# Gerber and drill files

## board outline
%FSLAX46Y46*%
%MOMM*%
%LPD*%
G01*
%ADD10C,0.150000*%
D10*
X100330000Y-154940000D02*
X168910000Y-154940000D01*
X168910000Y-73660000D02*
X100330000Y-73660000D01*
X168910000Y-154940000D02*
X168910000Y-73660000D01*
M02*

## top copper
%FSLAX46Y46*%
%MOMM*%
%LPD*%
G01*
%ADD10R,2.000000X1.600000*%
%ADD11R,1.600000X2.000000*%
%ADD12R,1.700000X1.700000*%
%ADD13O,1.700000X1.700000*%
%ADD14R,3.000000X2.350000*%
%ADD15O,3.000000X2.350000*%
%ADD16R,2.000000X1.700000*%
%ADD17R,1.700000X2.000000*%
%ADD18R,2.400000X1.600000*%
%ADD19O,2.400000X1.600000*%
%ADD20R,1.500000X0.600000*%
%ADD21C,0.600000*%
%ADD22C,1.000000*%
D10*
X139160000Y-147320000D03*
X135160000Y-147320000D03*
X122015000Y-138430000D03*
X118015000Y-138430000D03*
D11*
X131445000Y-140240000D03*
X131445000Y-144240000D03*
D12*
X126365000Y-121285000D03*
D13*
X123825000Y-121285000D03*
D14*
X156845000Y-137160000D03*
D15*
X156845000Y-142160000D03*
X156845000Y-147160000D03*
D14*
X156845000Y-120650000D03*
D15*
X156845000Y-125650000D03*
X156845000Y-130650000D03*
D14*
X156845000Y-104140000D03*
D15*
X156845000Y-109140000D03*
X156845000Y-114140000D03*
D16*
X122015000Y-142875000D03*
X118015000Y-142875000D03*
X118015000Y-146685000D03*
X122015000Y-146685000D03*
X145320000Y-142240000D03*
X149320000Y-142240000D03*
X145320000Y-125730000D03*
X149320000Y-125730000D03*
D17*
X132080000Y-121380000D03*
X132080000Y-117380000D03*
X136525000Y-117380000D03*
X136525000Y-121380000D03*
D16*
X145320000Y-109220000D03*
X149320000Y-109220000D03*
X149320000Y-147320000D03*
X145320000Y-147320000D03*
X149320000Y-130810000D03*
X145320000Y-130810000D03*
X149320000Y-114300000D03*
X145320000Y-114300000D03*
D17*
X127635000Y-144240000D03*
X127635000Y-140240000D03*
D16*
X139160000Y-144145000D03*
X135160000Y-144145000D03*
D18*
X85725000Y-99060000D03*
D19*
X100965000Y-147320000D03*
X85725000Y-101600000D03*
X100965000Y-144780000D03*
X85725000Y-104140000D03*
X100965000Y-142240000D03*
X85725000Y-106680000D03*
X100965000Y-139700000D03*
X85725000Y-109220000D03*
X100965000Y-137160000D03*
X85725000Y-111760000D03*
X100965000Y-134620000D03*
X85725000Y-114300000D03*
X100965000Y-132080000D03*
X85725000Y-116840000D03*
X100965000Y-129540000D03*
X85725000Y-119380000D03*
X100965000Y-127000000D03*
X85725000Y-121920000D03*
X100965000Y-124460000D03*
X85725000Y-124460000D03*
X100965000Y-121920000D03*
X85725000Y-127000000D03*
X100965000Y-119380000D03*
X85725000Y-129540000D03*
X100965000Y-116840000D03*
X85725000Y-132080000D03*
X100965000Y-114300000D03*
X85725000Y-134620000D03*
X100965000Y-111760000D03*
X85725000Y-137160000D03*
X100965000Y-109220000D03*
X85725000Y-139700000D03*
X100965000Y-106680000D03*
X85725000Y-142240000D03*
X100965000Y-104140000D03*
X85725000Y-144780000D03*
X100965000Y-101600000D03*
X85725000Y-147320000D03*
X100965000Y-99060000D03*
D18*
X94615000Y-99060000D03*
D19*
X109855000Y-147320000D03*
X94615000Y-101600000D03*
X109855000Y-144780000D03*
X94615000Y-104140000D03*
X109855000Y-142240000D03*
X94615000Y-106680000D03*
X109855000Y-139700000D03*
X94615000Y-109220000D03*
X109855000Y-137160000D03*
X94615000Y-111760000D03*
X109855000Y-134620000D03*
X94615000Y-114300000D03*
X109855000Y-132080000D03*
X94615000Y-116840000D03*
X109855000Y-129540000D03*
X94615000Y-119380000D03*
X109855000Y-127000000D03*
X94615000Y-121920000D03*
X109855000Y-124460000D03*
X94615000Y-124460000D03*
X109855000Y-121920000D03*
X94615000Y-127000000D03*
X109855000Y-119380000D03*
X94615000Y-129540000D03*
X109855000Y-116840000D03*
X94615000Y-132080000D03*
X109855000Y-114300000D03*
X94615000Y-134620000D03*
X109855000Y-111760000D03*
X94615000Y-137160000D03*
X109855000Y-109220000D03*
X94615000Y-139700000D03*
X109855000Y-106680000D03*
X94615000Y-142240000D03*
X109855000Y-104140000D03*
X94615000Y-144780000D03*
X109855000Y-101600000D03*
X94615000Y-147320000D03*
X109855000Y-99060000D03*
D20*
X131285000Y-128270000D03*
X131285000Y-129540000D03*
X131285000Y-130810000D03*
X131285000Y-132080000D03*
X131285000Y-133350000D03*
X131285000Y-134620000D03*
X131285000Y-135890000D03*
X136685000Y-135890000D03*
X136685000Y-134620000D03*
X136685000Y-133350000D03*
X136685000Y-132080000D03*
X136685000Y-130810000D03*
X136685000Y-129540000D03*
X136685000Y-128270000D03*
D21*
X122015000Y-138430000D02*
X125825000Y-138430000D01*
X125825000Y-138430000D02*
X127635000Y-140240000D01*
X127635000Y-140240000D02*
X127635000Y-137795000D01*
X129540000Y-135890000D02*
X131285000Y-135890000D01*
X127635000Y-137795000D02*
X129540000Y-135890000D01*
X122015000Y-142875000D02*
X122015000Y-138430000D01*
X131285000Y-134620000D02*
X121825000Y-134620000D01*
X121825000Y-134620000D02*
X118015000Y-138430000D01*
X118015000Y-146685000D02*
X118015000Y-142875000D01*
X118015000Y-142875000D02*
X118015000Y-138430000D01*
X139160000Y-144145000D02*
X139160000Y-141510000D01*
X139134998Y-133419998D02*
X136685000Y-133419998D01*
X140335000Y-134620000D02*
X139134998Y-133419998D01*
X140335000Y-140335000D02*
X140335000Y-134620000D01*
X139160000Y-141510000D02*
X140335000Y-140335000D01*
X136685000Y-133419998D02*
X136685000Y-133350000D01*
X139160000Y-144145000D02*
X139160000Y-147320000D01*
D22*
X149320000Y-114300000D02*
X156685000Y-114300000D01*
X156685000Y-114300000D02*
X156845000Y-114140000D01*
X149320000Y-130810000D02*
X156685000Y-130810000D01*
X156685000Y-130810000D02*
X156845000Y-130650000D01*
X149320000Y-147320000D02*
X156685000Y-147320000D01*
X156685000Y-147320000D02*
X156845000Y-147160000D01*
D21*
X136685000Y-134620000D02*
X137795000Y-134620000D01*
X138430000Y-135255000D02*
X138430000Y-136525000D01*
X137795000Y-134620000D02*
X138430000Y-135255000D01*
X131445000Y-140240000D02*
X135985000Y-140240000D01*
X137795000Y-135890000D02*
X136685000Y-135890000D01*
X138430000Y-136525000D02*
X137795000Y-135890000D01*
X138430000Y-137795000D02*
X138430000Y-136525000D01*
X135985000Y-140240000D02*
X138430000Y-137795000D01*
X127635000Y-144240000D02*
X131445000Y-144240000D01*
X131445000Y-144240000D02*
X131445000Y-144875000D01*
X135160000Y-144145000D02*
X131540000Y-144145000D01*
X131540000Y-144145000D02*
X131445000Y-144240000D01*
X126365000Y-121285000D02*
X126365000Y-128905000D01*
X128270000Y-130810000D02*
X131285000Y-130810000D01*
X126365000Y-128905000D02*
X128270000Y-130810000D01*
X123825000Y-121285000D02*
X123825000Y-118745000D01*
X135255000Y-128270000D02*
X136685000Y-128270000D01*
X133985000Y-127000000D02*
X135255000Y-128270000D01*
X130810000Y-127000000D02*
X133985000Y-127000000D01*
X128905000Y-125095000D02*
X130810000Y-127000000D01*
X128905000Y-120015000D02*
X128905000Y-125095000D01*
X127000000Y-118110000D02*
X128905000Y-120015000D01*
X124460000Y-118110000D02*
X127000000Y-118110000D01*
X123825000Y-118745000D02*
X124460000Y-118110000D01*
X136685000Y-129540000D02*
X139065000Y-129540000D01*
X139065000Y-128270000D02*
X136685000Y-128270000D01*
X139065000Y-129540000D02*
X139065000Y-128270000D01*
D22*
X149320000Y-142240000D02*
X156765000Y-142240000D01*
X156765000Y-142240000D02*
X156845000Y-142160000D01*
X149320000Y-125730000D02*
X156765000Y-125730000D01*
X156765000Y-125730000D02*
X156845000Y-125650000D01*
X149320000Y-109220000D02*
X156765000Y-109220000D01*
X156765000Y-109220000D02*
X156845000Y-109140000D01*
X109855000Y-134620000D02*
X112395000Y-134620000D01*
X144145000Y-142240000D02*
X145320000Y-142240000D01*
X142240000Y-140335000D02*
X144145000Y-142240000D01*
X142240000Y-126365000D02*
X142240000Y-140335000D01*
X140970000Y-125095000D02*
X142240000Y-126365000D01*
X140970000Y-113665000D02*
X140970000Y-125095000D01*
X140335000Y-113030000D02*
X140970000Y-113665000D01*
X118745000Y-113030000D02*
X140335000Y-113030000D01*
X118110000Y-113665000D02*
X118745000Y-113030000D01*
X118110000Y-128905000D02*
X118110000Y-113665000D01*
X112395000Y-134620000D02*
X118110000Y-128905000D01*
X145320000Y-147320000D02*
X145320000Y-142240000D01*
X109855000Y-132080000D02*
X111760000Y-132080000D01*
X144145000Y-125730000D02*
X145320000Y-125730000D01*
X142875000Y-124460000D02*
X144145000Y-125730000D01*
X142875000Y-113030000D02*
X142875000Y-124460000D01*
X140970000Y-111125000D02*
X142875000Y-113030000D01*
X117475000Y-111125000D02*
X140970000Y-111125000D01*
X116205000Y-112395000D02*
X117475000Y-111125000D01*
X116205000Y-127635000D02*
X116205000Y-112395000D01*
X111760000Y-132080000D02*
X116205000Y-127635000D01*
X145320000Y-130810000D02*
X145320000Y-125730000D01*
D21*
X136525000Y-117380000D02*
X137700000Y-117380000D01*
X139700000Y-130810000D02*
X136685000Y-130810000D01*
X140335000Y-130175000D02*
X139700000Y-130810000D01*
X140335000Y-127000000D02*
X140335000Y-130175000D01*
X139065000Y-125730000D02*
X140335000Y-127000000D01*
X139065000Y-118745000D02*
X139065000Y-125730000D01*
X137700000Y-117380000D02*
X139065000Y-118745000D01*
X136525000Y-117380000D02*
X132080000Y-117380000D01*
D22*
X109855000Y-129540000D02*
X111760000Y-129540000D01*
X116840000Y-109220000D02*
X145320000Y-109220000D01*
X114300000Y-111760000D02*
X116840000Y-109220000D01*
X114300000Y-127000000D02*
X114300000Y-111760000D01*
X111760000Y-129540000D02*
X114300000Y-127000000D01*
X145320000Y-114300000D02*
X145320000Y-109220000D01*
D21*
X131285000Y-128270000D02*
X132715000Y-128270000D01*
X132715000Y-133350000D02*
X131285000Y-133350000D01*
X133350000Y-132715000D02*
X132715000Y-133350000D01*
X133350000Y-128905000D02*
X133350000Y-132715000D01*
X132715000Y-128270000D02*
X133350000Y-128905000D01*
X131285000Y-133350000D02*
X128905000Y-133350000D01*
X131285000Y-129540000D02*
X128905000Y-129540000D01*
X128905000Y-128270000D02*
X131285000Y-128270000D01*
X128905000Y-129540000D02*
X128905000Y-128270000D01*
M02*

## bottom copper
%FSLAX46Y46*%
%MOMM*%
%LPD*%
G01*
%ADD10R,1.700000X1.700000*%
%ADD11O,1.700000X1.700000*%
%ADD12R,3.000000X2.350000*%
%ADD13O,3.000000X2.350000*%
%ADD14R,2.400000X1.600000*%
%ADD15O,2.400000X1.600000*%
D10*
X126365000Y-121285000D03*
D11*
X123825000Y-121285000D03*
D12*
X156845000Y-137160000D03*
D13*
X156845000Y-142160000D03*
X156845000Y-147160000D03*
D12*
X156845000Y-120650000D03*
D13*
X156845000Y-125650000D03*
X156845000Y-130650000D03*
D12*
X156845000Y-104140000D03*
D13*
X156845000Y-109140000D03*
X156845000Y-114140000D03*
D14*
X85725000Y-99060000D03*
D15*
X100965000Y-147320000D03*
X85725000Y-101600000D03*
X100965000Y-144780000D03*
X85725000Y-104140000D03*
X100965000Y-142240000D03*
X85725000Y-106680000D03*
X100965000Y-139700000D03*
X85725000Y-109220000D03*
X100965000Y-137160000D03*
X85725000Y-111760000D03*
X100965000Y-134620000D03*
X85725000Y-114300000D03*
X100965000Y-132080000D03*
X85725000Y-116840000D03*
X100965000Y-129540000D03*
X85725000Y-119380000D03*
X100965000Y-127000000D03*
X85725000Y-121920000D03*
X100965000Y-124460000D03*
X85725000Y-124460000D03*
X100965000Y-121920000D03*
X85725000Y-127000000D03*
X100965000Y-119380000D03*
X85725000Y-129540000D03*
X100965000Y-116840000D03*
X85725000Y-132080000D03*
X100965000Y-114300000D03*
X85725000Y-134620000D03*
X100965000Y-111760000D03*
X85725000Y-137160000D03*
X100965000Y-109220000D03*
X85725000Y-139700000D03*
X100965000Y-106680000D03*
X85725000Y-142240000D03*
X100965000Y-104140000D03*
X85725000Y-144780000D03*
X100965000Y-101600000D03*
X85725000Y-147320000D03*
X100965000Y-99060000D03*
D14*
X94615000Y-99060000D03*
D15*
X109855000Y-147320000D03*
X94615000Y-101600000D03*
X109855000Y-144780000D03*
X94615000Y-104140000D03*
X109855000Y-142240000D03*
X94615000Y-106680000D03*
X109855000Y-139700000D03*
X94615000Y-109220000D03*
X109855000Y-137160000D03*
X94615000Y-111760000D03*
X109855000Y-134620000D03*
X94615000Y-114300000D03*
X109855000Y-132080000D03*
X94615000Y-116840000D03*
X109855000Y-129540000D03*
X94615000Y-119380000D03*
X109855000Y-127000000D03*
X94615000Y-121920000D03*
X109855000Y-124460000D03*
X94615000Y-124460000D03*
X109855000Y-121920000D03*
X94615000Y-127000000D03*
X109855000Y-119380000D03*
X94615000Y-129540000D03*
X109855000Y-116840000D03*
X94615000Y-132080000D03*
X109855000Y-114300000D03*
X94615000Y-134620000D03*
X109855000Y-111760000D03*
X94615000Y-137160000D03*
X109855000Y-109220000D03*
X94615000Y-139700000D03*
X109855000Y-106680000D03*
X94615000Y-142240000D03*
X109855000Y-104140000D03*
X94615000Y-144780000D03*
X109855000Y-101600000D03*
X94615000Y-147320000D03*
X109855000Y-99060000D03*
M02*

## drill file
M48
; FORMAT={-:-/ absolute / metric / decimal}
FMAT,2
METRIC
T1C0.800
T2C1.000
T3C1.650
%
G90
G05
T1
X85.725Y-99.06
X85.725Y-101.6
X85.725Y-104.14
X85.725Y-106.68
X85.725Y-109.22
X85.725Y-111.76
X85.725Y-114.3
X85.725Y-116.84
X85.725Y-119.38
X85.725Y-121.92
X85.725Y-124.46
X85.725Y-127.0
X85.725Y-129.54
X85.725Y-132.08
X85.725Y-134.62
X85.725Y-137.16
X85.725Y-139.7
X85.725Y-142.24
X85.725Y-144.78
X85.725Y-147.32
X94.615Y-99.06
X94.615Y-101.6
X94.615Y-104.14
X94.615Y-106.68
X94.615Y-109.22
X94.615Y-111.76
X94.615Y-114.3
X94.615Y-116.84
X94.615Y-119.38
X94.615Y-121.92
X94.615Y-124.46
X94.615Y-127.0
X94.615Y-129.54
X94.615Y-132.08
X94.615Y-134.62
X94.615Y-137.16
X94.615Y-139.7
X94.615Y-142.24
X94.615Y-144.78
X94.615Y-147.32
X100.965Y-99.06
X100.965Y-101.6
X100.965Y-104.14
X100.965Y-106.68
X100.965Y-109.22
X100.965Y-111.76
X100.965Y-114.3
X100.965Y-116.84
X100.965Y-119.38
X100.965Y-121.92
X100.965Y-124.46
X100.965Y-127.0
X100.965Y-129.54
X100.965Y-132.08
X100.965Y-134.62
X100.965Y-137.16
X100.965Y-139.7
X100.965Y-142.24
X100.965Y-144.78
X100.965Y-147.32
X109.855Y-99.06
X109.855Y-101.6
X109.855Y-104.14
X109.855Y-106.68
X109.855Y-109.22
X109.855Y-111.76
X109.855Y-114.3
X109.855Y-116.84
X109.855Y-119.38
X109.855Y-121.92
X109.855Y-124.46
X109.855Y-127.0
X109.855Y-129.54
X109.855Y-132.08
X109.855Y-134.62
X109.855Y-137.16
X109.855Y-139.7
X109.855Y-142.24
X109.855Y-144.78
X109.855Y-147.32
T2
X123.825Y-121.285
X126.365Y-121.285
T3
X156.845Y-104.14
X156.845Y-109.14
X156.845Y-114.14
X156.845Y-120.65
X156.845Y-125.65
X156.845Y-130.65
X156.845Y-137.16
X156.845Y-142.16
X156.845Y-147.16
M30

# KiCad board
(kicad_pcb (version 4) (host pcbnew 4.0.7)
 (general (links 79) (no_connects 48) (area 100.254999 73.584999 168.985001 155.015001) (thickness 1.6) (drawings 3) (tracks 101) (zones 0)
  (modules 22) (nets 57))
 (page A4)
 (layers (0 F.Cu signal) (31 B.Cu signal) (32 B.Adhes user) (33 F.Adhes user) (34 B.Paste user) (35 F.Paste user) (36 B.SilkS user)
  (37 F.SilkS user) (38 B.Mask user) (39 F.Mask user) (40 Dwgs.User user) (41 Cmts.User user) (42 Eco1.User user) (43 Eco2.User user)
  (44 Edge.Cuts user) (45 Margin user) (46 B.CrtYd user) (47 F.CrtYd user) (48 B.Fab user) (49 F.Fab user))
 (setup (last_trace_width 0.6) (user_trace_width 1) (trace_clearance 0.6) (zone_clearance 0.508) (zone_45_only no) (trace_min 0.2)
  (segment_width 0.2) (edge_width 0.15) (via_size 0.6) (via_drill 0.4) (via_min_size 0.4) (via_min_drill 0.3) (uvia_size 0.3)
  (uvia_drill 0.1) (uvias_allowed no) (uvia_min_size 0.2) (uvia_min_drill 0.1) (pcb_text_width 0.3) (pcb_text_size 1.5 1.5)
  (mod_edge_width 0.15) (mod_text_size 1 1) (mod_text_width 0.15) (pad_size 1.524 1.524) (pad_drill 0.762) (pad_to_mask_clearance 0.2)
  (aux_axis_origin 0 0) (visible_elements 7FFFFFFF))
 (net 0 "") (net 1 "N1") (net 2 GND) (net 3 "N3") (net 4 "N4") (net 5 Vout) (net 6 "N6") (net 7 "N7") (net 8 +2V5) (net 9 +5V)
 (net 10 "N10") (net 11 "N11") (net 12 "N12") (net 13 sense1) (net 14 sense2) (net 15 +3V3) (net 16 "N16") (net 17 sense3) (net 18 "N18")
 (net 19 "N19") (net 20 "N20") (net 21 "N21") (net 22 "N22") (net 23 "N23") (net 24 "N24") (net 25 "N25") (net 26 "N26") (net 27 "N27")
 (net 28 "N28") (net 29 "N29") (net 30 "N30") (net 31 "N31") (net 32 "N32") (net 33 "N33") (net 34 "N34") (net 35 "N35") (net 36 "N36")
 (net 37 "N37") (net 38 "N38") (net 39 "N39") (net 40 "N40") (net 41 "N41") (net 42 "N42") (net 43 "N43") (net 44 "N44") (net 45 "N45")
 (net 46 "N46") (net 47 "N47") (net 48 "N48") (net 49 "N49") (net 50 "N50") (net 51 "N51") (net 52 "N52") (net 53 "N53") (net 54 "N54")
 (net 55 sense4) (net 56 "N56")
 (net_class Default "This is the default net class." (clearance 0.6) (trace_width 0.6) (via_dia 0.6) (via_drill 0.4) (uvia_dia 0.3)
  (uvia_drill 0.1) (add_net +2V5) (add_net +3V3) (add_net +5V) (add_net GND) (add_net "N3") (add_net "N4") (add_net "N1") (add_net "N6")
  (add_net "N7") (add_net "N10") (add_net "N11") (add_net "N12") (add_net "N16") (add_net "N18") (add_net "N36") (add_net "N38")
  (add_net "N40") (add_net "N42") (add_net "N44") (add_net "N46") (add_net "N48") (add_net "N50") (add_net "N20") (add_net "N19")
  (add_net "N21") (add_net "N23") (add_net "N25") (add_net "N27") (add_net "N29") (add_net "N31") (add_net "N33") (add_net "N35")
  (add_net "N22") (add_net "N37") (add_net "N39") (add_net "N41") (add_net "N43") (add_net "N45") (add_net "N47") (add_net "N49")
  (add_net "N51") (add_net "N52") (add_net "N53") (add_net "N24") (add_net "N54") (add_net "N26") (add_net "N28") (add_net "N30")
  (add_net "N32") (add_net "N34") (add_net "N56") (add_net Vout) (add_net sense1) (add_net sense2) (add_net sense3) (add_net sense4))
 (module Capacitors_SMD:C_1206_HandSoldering (layer F.Cu) (at 137.16 147.32 180)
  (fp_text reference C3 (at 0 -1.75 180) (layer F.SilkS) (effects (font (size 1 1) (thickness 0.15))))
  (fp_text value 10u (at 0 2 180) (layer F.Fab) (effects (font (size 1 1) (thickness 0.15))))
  (pad 1 smd rect (at -2 0 180) (size 2 1.6) (layers F.Cu F.Paste F.Mask) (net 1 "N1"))
  (pad 2 smd rect (at 2 0 180) (size 2 1.6) (layers F.Cu F.Paste F.Mask) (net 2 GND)))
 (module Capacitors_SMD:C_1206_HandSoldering (layer F.Cu) (at 120.015 138.43 180)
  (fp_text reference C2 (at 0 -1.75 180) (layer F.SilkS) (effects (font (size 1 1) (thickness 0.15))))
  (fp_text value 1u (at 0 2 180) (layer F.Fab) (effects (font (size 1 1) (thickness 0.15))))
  (pad 1 smd rect (at -2 0 180) (size 2 1.6) (layers F.Cu F.Paste F.Mask) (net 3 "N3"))
  (pad 2 smd rect (at 2 0 180) (size 2 1.6) (layers F.Cu F.Paste F.Mask) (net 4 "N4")))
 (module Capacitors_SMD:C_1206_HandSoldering (layer F.Cu) (at 131.445 142.24 270)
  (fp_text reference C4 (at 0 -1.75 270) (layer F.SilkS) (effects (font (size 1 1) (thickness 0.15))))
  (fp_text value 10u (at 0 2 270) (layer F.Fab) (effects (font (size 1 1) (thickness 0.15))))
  (pad 1 smd rect (at -2 0 270) (size 2 1.6) (layers F.Cu F.Paste F.Mask) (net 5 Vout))
  (pad 2 smd rect (at 2 0 270) (size 2 1.6) (layers F.Cu F.Paste F.Mask) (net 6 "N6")))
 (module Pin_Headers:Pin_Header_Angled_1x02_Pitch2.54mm (layer B.Cu) (at 126.365 121.285 90)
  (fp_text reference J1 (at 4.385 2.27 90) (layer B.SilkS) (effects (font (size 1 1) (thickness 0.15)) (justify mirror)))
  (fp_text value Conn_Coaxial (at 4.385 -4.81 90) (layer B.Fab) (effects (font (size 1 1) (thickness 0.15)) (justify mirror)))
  (pad 1 thru_hole rect (at 0 0 90) (size 1.7 1.7) (drill 1) (layers *.Cu *.Mask) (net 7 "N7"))
  (pad 2 thru_hole oval (at 0 -2.54 90) (size 1.7 1.7) (drill 1) (layers *.Cu *.Mask) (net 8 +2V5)))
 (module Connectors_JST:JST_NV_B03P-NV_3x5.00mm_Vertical (layer F.Cu) (at 156.845 137.16 270)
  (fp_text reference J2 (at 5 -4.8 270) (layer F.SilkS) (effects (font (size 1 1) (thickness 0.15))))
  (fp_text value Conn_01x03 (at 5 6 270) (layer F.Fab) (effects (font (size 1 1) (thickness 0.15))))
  (pad 1 thru_hole rect (at 0 0 270) (size 2.35 3) (drill 1.65) (layers *.Cu *.Mask) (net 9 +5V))
  (pad 2 thru_hole oval (at 5 0 270) (size 2.35 3) (drill 1.65) (layers *.Cu *.Mask) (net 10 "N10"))
  (pad 3 thru_hole oval (at 10 0 270) (size 2.35 3) (drill 1.65) (layers *.Cu *.Mask) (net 2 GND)))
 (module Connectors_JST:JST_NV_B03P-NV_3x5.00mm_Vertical (layer F.Cu) (at 156.845 120.65 270)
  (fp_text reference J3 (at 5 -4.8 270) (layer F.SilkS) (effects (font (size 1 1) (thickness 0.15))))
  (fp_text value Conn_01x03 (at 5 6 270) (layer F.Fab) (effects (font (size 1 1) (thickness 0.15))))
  (pad 1 thru_hole rect (at 0 0 270) (size 2.35 3) (drill 1.65) (layers *.Cu *.Mask) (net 9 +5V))
  (pad 2 thru_hole oval (at 5 0 270) (size 2.35 3) (drill 1.65) (layers *.Cu *.Mask) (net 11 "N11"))
  (pad 3 thru_hole oval (at 10 0 270) (size 2.35 3) (drill 1.65) (layers *.Cu *.Mask) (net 2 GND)))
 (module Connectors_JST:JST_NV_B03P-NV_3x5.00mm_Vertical (layer F.Cu) (at 156.845 104.14 270)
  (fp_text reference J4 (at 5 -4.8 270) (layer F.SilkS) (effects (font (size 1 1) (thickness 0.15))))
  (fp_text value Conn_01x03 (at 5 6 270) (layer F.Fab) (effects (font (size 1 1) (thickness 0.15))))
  (pad 1 thru_hole rect (at 0 0 270) (size 2.35 3) (drill 1.65) (layers *.Cu *.Mask) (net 9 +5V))
  (pad 2 thru_hole oval (at 5 0 270) (size 2.35 3) (drill 1.65) (layers *.Cu *.Mask) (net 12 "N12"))
  (pad 3 thru_hole oval (at 10 0 270) (size 2.35 3) (drill 1.65) (layers *.Cu *.Mask) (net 2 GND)))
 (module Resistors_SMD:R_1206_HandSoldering (layer F.Cu) (at 120.015 142.875 180)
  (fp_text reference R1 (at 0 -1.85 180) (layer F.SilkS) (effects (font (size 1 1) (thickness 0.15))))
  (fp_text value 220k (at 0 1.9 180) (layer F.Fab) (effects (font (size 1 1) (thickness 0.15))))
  (pad 1 smd rect (at -2 0 180) (size 2 1.7) (layers F.Cu F.Paste F.Mask) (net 3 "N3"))
  (pad 2 smd rect (at 2 0 180) (size 2 1.7) (layers F.Cu F.Paste F.Mask) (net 4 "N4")))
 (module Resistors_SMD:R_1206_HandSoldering (layer F.Cu) (at 120.015 146.685)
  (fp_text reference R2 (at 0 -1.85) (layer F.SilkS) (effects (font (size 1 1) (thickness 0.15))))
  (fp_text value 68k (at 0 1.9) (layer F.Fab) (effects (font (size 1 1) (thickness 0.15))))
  (pad 1 smd rect (at -2 0) (size 2 1.7) (layers F.Cu F.Paste F.Mask) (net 4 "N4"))
  (pad 2 smd rect (at 2 0) (size 2 1.7) (layers F.Cu F.Paste F.Mask) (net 8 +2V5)))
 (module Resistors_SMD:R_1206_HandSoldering (layer F.Cu) (at 147.32 142.24)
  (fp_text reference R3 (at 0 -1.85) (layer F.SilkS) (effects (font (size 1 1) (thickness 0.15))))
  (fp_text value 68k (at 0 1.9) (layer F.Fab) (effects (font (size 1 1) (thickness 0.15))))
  (pad 1 smd rect (at -2 0) (size 2 1.7) (layers F.Cu F.Paste F.Mask) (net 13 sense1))
  (pad 2 smd rect (at 2 0) (size 2 1.7) (layers F.Cu F.Paste F.Mask) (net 10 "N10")))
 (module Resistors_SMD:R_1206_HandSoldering (layer F.Cu) (at 147.32 125.73)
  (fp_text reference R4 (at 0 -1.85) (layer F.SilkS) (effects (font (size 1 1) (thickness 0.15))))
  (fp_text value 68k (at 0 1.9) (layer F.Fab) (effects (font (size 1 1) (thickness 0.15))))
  (pad 1 smd rect (at -2 0) (size 2 1.7) (layers F.Cu F.Paste F.Mask) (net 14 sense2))
  (pad 2 smd rect (at 2 0) (size 2 1.7) (layers F.Cu F.Paste F.Mask) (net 11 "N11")))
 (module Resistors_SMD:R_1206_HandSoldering (layer F.Cu) (at 132.08 119.38 90)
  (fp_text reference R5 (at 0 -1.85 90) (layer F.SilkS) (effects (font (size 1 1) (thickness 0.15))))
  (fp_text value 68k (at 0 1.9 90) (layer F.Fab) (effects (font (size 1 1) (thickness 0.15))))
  (pad 1 smd rect (at -2 0 90) (size 2 1.7) (layers F.Cu F.Paste F.Mask) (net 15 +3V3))
  (pad 2 smd rect (at 2 0 90) (size 2 1.7) (layers F.Cu F.Paste F.Mask) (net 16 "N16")))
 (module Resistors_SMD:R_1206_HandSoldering (layer F.Cu) (at 136.525 119.38 270)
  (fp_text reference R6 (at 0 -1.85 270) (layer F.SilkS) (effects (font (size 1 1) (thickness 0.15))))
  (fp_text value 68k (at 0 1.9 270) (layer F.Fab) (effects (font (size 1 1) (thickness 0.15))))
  (pad 1 smd rect (at -2 0 270) (size 2 1.7) (layers F.Cu F.Paste F.Mask) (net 16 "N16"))
  (pad 2 smd rect (at 2 0 270) (size 2 1.7) (layers F.Cu F.Paste F.Mask) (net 2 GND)))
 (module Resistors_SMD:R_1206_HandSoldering (layer F.Cu) (at 147.32 109.22)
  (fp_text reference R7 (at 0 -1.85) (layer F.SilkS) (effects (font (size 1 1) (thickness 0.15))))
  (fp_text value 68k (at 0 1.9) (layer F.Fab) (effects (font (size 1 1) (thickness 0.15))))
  (pad 1 smd rect (at -2 0) (size 2 1.7) (layers F.Cu F.Paste F.Mask) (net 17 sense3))
  (pad 2 smd rect (at 2 0) (size 2 1.7) (layers F.Cu F.Paste F.Mask) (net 12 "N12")))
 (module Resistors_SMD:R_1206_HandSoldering (layer F.Cu) (at 147.32 147.32 180)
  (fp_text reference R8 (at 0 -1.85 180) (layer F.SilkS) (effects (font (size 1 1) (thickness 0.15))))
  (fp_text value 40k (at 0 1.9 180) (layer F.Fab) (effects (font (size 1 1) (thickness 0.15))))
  (pad 1 smd rect (at -2 0 180) (size 2 1.7) (layers F.Cu F.Paste F.Mask) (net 2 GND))
  (pad 2 smd rect (at 2 0 180) (size 2 1.7) (layers F.Cu F.Paste F.Mask) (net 13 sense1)))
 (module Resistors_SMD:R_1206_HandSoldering (layer F.Cu) (at 147.32 130.81 180)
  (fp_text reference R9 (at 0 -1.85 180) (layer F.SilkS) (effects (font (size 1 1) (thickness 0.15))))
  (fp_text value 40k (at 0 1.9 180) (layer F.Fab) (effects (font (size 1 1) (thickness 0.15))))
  (pad 1 smd rect (at -2 0 180) (size 2 1.7) (layers F.Cu F.Paste F.Mask) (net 2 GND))
  (pad 2 smd rect (at 2 0 180) (size 2 1.7) (layers F.Cu F.Paste F.Mask) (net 14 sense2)))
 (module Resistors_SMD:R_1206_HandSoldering (layer F.Cu) (at 147.32 114.3 180)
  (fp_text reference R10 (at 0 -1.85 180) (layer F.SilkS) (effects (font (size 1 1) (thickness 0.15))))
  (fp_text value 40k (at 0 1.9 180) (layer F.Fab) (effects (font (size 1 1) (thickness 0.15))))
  (pad 1 smd rect (at -2 0 180) (size 2 1.7) (layers F.Cu F.Paste F.Mask) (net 2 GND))
  (pad 2 smd rect (at 2 0 180) (size 2 1.7) (layers F.Cu F.Paste F.Mask) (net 17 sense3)))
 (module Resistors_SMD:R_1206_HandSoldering (layer F.Cu) (at 127.635 142.24 90)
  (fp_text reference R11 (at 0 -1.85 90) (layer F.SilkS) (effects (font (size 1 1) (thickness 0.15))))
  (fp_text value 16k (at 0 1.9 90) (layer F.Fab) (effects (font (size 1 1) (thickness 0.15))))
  (pad 1 smd rect (at -2 0 90) (size 2 1.7) (layers F.Cu F.Paste F.Mask) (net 6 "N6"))
  (pad 2 smd rect (at 2 0 90) (size 2 1.7) (layers F.Cu F.Paste F.Mask) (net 3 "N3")))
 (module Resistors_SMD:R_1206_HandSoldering (layer F.Cu) (at 137.16 144.145 180)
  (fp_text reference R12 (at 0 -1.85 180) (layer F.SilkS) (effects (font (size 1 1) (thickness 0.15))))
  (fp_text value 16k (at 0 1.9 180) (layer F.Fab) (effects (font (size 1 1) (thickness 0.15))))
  (pad 1 smd rect (at -2 0 180) (size 2 1.7) (layers F.Cu F.Paste F.Mask) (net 1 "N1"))
  (pad 2 smd rect (at 2 0 180) (size 2 1.7) (layers F.Cu F.Paste F.Mask) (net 6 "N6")))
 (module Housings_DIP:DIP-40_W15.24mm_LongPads (layer F.Cu) (at 85.725 99.06)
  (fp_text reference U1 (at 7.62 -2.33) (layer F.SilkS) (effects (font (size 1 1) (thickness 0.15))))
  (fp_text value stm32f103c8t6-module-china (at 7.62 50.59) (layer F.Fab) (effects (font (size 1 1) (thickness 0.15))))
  (pad 1 thru_hole rect (at 0 0) (size 2.4 1.6) (drill 0.8) (layers *.Cu *.Mask) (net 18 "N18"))
  (pad 21 thru_hole oval (at 15.24 48.26) (size 2.4 1.6) (drill 0.8) (layers *.Cu *.Mask) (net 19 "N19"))
  (pad 2 thru_hole oval (at 0 2.54) (size 2.4 1.6) (drill 0.8) (layers *.Cu *.Mask) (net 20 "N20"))
  (pad 22 thru_hole oval (at 15.24 45.72) (size 2.4 1.6) (drill 0.8) (layers *.Cu *.Mask) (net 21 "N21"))
  (pad 3 thru_hole oval (at 0 5.08) (size 2.4 1.6) (drill 0.8) (layers *.Cu *.Mask) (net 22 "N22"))
  (pad 23 thru_hole oval (at 15.24 43.18) (size 2.4 1.6) (drill 0.8) (layers *.Cu *.Mask) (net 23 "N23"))
  (pad 4 thru_hole oval (at 0 7.62) (size 2.4 1.6) (drill 0.8) (layers *.Cu *.Mask) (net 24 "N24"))
  (pad 24 thru_hole oval (at 15.24 40.64) (size 2.4 1.6) (drill 0.8) (layers *.Cu *.Mask) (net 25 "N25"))
  (pad 5 thru_hole oval (at 0 10.16) (size 2.4 1.6) (drill 0.8) (layers *.Cu *.Mask) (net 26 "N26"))
  (pad 25 thru_hole oval (at 15.24 38.1) (size 2.4 1.6) (drill 0.8) (layers *.Cu *.Mask) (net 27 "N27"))
  (pad 6 thru_hole oval (at 0 12.7) (size 2.4 1.6) (drill 0.8) (layers *.Cu *.Mask) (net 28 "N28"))
  (pad 26 thru_hole oval (at 15.24 35.56) (size 2.4 1.6) (drill 0.8) (layers *.Cu *.Mask) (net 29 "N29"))
  (pad 7 thru_hole oval (at 0 15.24) (size 2.4 1.6) (drill 0.8) (layers *.Cu *.Mask) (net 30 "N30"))
  (pad 27 thru_hole oval (at 15.24 33.02) (size 2.4 1.6) (drill 0.8) (layers *.Cu *.Mask) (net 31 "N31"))
  (pad 8 thru_hole oval (at 0 17.78) (size 2.4 1.6) (drill 0.8) (layers *.Cu *.Mask) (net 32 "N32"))
  (pad 28 thru_hole oval (at 15.24 30.48) (size 2.4 1.6) (drill 0.8) (layers *.Cu *.Mask) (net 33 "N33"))
  (pad 9 thru_hole oval (at 0 20.32) (size 2.4 1.6) (drill 0.8) (layers *.Cu *.Mask) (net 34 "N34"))
  (pad 29 thru_hole oval (at 15.24 27.94) (size 2.4 1.6) (drill 0.8) (layers *.Cu *.Mask) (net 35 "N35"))
  (pad 10 thru_hole oval (at 0 22.86) (size 2.4 1.6) (drill 0.8) (layers *.Cu *.Mask) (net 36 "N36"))
  (pad 30 thru_hole oval (at 15.24 25.4) (size 2.4 1.6) (drill 0.8) (layers *.Cu *.Mask) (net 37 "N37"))
  (pad 11 thru_hole oval (at 0 25.4) (size 2.4 1.6) (drill 0.8) (layers *.Cu *.Mask) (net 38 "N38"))
  (pad 31 thru_hole oval (at 15.24 22.86) (size 2.4 1.6) (drill 0.8) (layers *.Cu *.Mask) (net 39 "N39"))
  (pad 12 thru_hole oval (at 0 27.94) (size 2.4 1.6) (drill 0.8) (layers *.Cu *.Mask) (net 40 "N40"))
  (pad 32 thru_hole oval (at 15.24 20.32) (size 2.4 1.6) (drill 0.8) (layers *.Cu *.Mask) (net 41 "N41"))
  (pad 13 thru_hole oval (at 0 30.48) (size 2.4 1.6) (drill 0.8) (layers *.Cu *.Mask) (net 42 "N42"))
  (pad 33 thru_hole oval (at 15.24 17.78) (size 2.4 1.6) (drill 0.8) (layers *.Cu *.Mask) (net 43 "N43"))
  (pad 14 thru_hole oval (at 0 33.02) (size 2.4 1.6) (drill 0.8) (layers *.Cu *.Mask) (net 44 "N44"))
  (pad 34 thru_hole oval (at 15.24 15.24) (size 2.4 1.6) (drill 0.8) (layers *.Cu *.Mask) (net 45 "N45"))
  (pad 15 thru_hole oval (at 0 35.56) (size 2.4 1.6) (drill 0.8) (layers *.Cu *.Mask) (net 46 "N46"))
  (pad 35 thru_hole oval (at 15.24 12.7) (size 2.4 1.6) (drill 0.8) (layers *.Cu *.Mask) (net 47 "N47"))
  (pad 16 thru_hole oval (at 0 38.1) (size 2.4 1.6) (drill 0.8) (layers *.Cu *.Mask) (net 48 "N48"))
  (pad 36 thru_hole oval (at 15.24 10.16) (size 2.4 1.6) (drill 0.8) (layers *.Cu *.Mask) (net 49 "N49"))
  (pad 17 thru_hole oval (at 0 40.64) (size 2.4 1.6) (drill 0.8) (layers *.Cu *.Mask) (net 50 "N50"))
  (pad 37 thru_hole oval (at 15.24 7.62) (size 2.4 1.6) (drill 0.8) (layers *.Cu *.Mask) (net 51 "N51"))
  (pad 18 thru_hole oval (at 0 43.18) (size 2.4 1.6) (drill 0.8) (layers *.Cu *.Mask) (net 9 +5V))
  (pad 38 thru_hole oval (at 15.24 5.08) (size 2.4 1.6) (drill 0.8) (layers *.Cu *.Mask) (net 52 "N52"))
  (pad 19 thru_hole oval (at 0 45.72) (size 2.4 1.6) (drill 0.8) (layers *.Cu *.Mask) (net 2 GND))
  (pad 39 thru_hole oval (at 15.24 2.54) (size 2.4 1.6) (drill 0.8) (layers *.Cu *.Mask) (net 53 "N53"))
  (pad 20 thru_hole oval (at 0 48.26) (size 2.4 1.6) (drill 0.8) (layers *.Cu *.Mask) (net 15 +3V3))
  (pad 40 thru_hole oval (at 15.24 0) (size 2.4 1.6) (drill 0.8) (layers *.Cu *.Mask) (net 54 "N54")))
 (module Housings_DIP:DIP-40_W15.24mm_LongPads (layer F.Cu) (at 94.615 99.06)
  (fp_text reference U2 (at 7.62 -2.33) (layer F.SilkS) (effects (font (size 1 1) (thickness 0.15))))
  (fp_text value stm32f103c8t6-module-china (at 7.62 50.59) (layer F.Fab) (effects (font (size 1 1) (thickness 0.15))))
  (pad 1 thru_hole rect (at 0 0) (size 2.4 1.6) (drill 0.8) (layers *.Cu *.Mask) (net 18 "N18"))
  (pad 21 thru_hole oval (at 15.24 48.26) (size 2.4 1.6) (drill 0.8) (layers *.Cu *.Mask) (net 19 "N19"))
  (pad 2 thru_hole oval (at 0 2.54) (size 2.4 1.6) (drill 0.8) (layers *.Cu *.Mask) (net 20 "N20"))
  (pad 22 thru_hole oval (at 15.24 45.72) (size 2.4 1.6) (drill 0.8) (layers *.Cu *.Mask) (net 21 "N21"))
  (pad 3 thru_hole oval (at 0 5.08) (size 2.4 1.6) (drill 0.8) (layers *.Cu *.Mask) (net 22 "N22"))
  (pad 23 thru_hole oval (at 15.24 43.18) (size 2.4 1.6) (drill 0.8) (layers *.Cu *.Mask) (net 23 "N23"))
  (pad 4 thru_hole oval (at 0 7.62) (size 2.4 1.6) (drill 0.8) (layers *.Cu *.Mask) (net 24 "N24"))
  (pad 24 thru_hole oval (at 15.24 40.64) (size 2.4 1.6) (drill 0.8) (layers *.Cu *.Mask) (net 25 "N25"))
  (pad 5 thru_hole oval (at 0 10.16) (size 2.4 1.6) (drill 0.8) (layers *.Cu *.Mask) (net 26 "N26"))
  (pad 25 thru_hole oval (at 15.24 38.1) (size 2.4 1.6) (drill 0.8) (layers *.Cu *.Mask) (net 5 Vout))
  (pad 6 thru_hole oval (at 0 12.7) (size 2.4 1.6) (drill 0.8) (layers *.Cu *.Mask) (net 28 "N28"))
  (pad 26 thru_hole oval (at 15.24 35.56) (size 2.4 1.6) (drill 0.8) (layers *.Cu *.Mask) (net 13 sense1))
  (pad 7 thru_hole oval (at 0 15.24) (size 2.4 1.6) (drill 0.8) (layers *.Cu *.Mask) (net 30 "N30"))
  (pad 27 thru_hole oval (at 15.24 33.02) (size 2.4 1.6) (drill 0.8) (layers *.Cu *.Mask) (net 14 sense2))
  (pad 8 thru_hole oval (at 0 17.78) (size 2.4 1.6) (drill 0.8) (layers *.Cu *.Mask) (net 32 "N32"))
  (pad 28 thru_hole oval (at 15.24 30.48) (size 2.4 1.6) (drill 0.8) (layers *.Cu *.Mask) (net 17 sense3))
  (pad 9 thru_hole oval (at 0 20.32) (size 2.4 1.6) (drill 0.8) (layers *.Cu *.Mask) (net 34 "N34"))
  (pad 29 thru_hole oval (at 15.24 27.94) (size 2.4 1.6) (drill 0.8) (layers *.Cu *.Mask) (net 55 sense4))
  (pad 10 thru_hole oval (at 0 22.86) (size 2.4 1.6) (drill 0.8) (layers *.Cu *.Mask) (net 36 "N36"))
  (pad 30 thru_hole oval (at 15.24 25.4) (size 2.4 1.6) (drill 0.8) (layers *.Cu *.Mask) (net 37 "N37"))
  (pad 11 thru_hole oval (at 0 25.4) (size 2.4 1.6) (drill 0.8) (layers *.Cu *.Mask) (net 38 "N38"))
  (pad 31 thru_hole oval (at 15.24 22.86) (size 2.4 1.6) (drill 0.8) (layers *.Cu *.Mask) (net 39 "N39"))
  (pad 12 thru_hole oval (at 0 27.94) (size 2.4 1.6) (drill 0.8) (layers *.Cu *.Mask) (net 40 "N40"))
  (pad 32 thru_hole oval (at 15.24 20.32) (size 2.4 1.6) (drill 0.8) (layers *.Cu *.Mask) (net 41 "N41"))
  (pad 13 thru_hole oval (at 0 30.48) (size 2.4 1.6) (drill 0.8) (layers *.Cu *.Mask) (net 42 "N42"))
  (pad 33 thru_hole oval (at 15.24 17.78) (size 2.4 1.6) (drill 0.8) (layers *.Cu *.Mask) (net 43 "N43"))
  (pad 14 thru_hole oval (at 0 33.02) (size 2.4 1.6) (drill 0.8) (layers *.Cu *.Mask) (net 44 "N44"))
  (pad 34 thru_hole oval (at 15.24 15.24) (size 2.4 1.6) (drill 0.8) (layers *.Cu *.Mask) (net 45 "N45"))
  (pad 15 thru_hole oval (at 0 35.56) (size 2.4 1.6) (drill 0.8) (layers *.Cu *.Mask) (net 46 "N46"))
  (pad 35 thru_hole oval (at 15.24 12.7) (size 2.4 1.6) (drill 0.8) (layers *.Cu *.Mask) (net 47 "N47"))
  (pad 16 thru_hole oval (at 0 38.1) (size 2.4 1.6) (drill 0.8) (layers *.Cu *.Mask) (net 48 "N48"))
  (pad 36 thru_hole oval (at 15.24 10.16) (size 2.4 1.6) (drill 0.8) (layers *.Cu *.Mask) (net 49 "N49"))
  (pad 17 thru_hole oval (at 0 40.64) (size 2.4 1.6) (drill 0.8) (layers *.Cu *.Mask) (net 50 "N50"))
  (pad 37 thru_hole oval (at 15.24 7.62) (size 2.4 1.6) (drill 0.8) (layers *.Cu *.Mask) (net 51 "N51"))
  (pad 18 thru_hole oval (at 0 43.18) (size 2.4 1.6) (drill 0.8) (layers *.Cu *.Mask) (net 9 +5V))
  (pad 38 thru_hole oval (at 15.24 5.08) (size 2.4 1.6) (drill 0.8) (layers *.Cu *.Mask) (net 52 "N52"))
  (pad 19 thru_hole oval (at 0 45.72) (size 2.4 1.6) (drill 0.8) (layers *.Cu *.Mask) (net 2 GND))
  (pad 39 thru_hole oval (at 15.24 2.54) (size 2.4 1.6) (drill 0.8) (layers *.Cu *.Mask) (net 53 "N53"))
  (pad 20 thru_hole oval (at 0 48.26) (size 2.4 1.6) (drill 0.8) (layers *.Cu *.Mask) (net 15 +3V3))
  (pad 40 thru_hole oval (at 15.24 0) (size 2.4 1.6) (drill 0.8) (layers *.Cu *.Mask) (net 54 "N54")))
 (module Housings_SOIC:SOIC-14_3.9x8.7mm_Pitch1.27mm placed (layer F.Cu) (at 133.985 132.08)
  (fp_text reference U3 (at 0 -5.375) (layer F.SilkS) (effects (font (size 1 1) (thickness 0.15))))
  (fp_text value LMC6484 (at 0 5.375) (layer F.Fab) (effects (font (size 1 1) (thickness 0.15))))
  (pad 1 smd rect (at -2.7 -3.81) (size 1.5 0.6) (layers F.Cu F.Paste F.Mask) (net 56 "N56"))
  (pad 2 smd rect (at -2.7 -2.54) (size 1.5 0.6) (layers F.Cu F.Paste F.Mask) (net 56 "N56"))
  (pad 3 smd rect (at -2.7 -1.27) (size 1.5 0.6) (layers F.Cu F.Paste F.Mask) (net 7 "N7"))
  (pad 4 smd rect (at -2.7 0) (size 1.5 0.6) (layers F.Cu F.Paste F.Mask) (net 9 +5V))
  (pad 5 smd rect (at -2.7 1.27) (size 1.5 0.6) (layers F.Cu F.Paste F.Mask) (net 56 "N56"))
  (pad 6 smd rect (at -2.7 2.54) (size 1.5 0.6) (layers F.Cu F.Paste F.Mask) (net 4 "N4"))
  (pad 7 smd rect (at -2.7 3.81) (size 1.5 0.6) (layers F.Cu F.Paste F.Mask) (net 3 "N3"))
  (pad 8 smd rect (at 2.7 3.81) (size 1.5 0.6) (layers F.Cu F.Paste F.Mask) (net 5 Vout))
  (pad 9 smd rect (at 2.7 2.54) (size 1.5 0.6) (layers F.Cu F.Paste F.Mask) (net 5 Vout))
  (pad 10 smd rect (at 2.7 1.27) (size 1.5 0.6) (layers F.Cu F.Paste F.Mask) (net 1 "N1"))
  (pad 11 smd rect (at 2.7 0) (size 1.5 0.6) (layers F.Cu F.Paste F.Mask) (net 2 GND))
  (pad 12 smd rect (at 2.7 -1.27) (size 1.5 0.6) (layers F.Cu F.Paste F.Mask) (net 16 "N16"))
  (pad 13 smd rect (at 2.7 -2.54) (size 1.5 0.6) (layers F.Cu F.Paste F.Mask) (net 8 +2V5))
  (pad 14 smd rect (at 2.7 -3.81) (size 1.5 0.6) (layers F.Cu F.Paste F.Mask) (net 8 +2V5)))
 (gr_line (start 100.33 154.94) (end 168.91 154.94) (angle 90) (layer Edge.Cuts) (width 0.15))
 (gr_line (start 168.91 73.66) (end 100.33 73.66) (angle 90) (layer Edge.Cuts) (width 0.15))
 (gr_line (start 168.91 154.94) (end 168.91 73.66) (angle 90) (layer Edge.Cuts) (width 0.15))
 (segment (start 122.015 138.43) (end 125.825 138.43) (width 0.6) (layer F.Cu) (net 3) (status 400000))
 (segment (start 125.825 138.43) (end 127.635 140.24) (width 0.6) (layer F.Cu) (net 3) (status 800000))
 (segment (start 127.635 140.24) (end 127.635 137.795) (width 0.6) (layer F.Cu) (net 3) (status 400000))
 (segment (start 129.54 135.89) (end 131.285 135.89) (width 0.6) (layer F.Cu) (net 3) (status 800000))
 (segment (start 127.635 137.795) (end 129.54 135.89) (width 0.6) (layer F.Cu) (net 3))
 (segment (start 122.015 142.875) (end 122.015 138.43) (width 0.6) (layer F.Cu) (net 3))
 (segment (start 131.285 134.62) (end 121.825 134.62) (width 0.6) (layer F.Cu) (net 4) (status 400000))
 (segment (start 121.825 134.62) (end 118.015 138.43) (width 0.6) (layer F.Cu) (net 4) (status 800000))
 (segment (start 118.015 146.685) (end 118.015 142.875) (width 0.6) (layer F.Cu) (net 4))
 (segment (start 118.015 142.875) (end 118.015 138.43) (width 0.6) (layer F.Cu) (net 4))
 (segment (start 139.16 144.145) (end 139.16 141.51) (width 0.6) (layer F.Cu) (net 1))
 (segment (start 139.134998 133.419998) (end 136.685 133.419998) (width 0.6) (layer F.Cu) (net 1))
 (segment (start 140.335 134.62) (end 139.134998 133.419998) (width 0.6) (layer F.Cu) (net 1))
 (segment (start 140.335 140.335) (end 140.335 134.62) (width 0.6) (layer F.Cu) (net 1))
 (segment (start 139.16 141.51) (end 140.335 140.335) (width 0.6) (layer F.Cu) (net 1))
 (segment (start 136.685 133.419998) (end 136.685 133.35) (width 0.6) (layer F.Cu) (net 1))
 (segment (start 139.16 144.145) (end 139.16 147.32) (width 0.6) (layer F.Cu) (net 1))
 (segment (start 149.32 114.3) (end 156.685 114.3) (width 1) (layer F.Cu) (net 2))
 (segment (start 156.685 114.3) (end 156.845 114.14) (width 1) (layer F.Cu) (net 2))
 (segment (start 149.32 130.81) (end 156.685 130.81) (width 1) (layer F.Cu) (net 2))
 (segment (start 156.685 130.81) (end 156.845 130.65) (width 1) (layer F.Cu) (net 2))
 (segment (start 149.32 147.32) (end 156.685 147.32) (width 1) (layer F.Cu) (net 2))
 (segment (start 156.685 147.32) (end 156.845 147.16) (width 1) (layer F.Cu) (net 2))
 (segment (start 136.685 134.62) (end 137.795 134.62) (width 0.6) (layer F.Cu) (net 5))
 (segment (start 138.43 135.255) (end 138.43 136.525) (width 0.6) (layer F.Cu) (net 5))
 (segment (start 137.795 134.62) (end 138.43 135.255) (width 0.6) (layer F.Cu) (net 5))
 (segment (start 131.445 140.24) (end 135.985 140.24) (width 0.6) (layer F.Cu) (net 5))
 (segment (start 137.795 135.89) (end 136.685 135.89) (width 0.6) (layer F.Cu) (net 5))
 (segment (start 138.43 136.525) (end 137.795 135.89) (width 0.6) (layer F.Cu) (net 5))
 (segment (start 138.43 137.795) (end 138.43 136.525) (width 0.6) (layer F.Cu) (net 5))
 (segment (start 135.985 140.24) (end 138.43 137.795) (width 0.6) (layer F.Cu) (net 5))
 (segment (start 127.635 144.24) (end 131.445 144.24) (width 0.6) (layer F.Cu) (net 6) (status C00000))
 (segment (start 131.445 144.24) (end 131.445 144.875) (width 0.6) (layer F.Cu) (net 6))
 (segment (start 135.16 144.145) (end 131.54 144.145) (width 0.6) (layer F.Cu) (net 6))
 (segment (start 131.54 144.145) (end 131.445 144.24) (width 0.6) (layer F.Cu) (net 6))
 (segment (start 126.365 121.285) (end 126.365 128.905) (width 0.6) (layer F.Cu) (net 7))
 (segment (start 128.27 130.81) (end 131.285 130.81) (width 0.6) (layer F.Cu) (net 7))
 (segment (start 126.365 128.905) (end 128.27 130.81) (width 0.6) (layer F.Cu) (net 7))
 (segment (start 123.825 121.285) (end 123.825 118.745) (width 0.6) (layer F.Cu) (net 8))
 (segment (start 135.255 128.27) (end 136.685 128.27) (width 0.6) (layer F.Cu) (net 8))
 (segment (start 133.985 127) (end 135.255 128.27) (width 0.6) (layer F.Cu) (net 8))
 (segment (start 130.81 127) (end 133.985 127) (width 0.6) (layer F.Cu) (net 8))
 (segment (start 128.905 125.095) (end 130.81 127) (width 0.6) (layer F.Cu) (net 8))
 (segment (start 128.905 120.015) (end 128.905 125.095) (width 0.6) (layer F.Cu) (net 8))
 (segment (start 127 118.11) (end 128.905 120.015) (width 0.6) (layer F.Cu) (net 8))
 (segment (start 124.46 118.11) (end 127 118.11) (width 0.6) (layer F.Cu) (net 8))
 (segment (start 123.825 118.745) (end 124.46 118.11) (width 0.6) (layer F.Cu) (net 8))
 (segment (start 136.685 129.54) (end 139.065 129.54) (width 0.6) (layer F.Cu) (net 8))
 (segment (start 139.065 128.27) (end 136.685 128.27) (width 0.6) (layer F.Cu) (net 8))
 (segment (start 139.065 129.54) (end 139.065 128.27) (width 0.6) (layer F.Cu) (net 8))
 (segment (start 149.32 142.24) (end 156.765 142.24) (width 1) (layer F.Cu) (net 10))
 (segment (start 156.765 142.24) (end 156.845 142.16) (width 1) (layer F.Cu) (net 10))
 (segment (start 149.32 125.73) (end 156.765 125.73) (width 1) (layer F.Cu) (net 11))
 (segment (start 156.765 125.73) (end 156.845 125.65) (width 1) (layer F.Cu) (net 11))
 (segment (start 149.32 109.22) (end 156.765 109.22) (width 1) (layer F.Cu) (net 12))
 (segment (start 156.765 109.22) (end 156.845 109.14) (width 1) (layer F.Cu) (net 12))
 (segment (start 109.855 134.62) (end 112.395 134.62) (width 1) (layer F.Cu) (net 13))
 (segment (start 144.145 142.24) (end 145.32 142.24) (width 1) (layer F.Cu) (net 13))
 (segment (start 142.24 140.335) (end 144.145 142.24) (width 1) (layer F.Cu) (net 13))
 (segment (start 142.24 126.365) (end 142.24 140.335) (width 1) (layer F.Cu) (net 13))
 (segment (start 140.97 125.095) (end 142.24 126.365) (width 1) (layer F.Cu) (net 13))
 (segment (start 140.97 113.665) (end 140.97 125.095) (width 1) (layer F.Cu) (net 13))
 (segment (start 140.335 113.03) (end 140.97 113.665) (width 1) (layer F.Cu) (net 13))
 (segment (start 118.745 113.03) (end 140.335 113.03) (width 1) (layer F.Cu) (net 13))
 (segment (start 118.11 113.665) (end 118.745 113.03) (width 1) (layer F.Cu) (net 13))
 (segment (start 118.11 128.905) (end 118.11 113.665) (width 1) (layer F.Cu) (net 13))
 (segment (start 112.395 134.62) (end 118.11 128.905) (width 1) (layer F.Cu) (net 13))
 (segment (start 145.32 147.32) (end 145.32 142.24) (width 1) (layer F.Cu) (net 13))
 (segment (start 109.855 132.08) (end 111.76 132.08) (width 1) (layer F.Cu) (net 14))
 (segment (start 144.145 125.73) (end 145.32 125.73) (width 1) (layer F.Cu) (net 14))
 (segment (start 142.875 124.46) (end 144.145 125.73) (width 1) (layer F.Cu) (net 14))
 (segment (start 142.875 113.03) (end 142.875 124.46) (width 1) (layer F.Cu) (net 14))
 (segment (start 140.97 111.125) (end 142.875 113.03) (width 1) (layer F.Cu) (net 14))
 (segment (start 117.475 111.125) (end 140.97 111.125) (width 1) (layer F.Cu) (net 14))
 (segment (start 116.205 112.395) (end 117.475 111.125) (width 1) (layer F.Cu) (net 14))
 (segment (start 116.205 127.635) (end 116.205 112.395) (width 1) (layer F.Cu) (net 14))
 (segment (start 111.76 132.08) (end 116.205 127.635) (width 1) (layer F.Cu) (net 14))
 (segment (start 145.32 130.81) (end 145.32 125.73) (width 1) (layer F.Cu) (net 14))
 (segment (start 136.525 117.38) (end 137.7 117.38) (width 0.6) (layer F.Cu) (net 16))
 (segment (start 139.7 130.81) (end 136.685 130.81) (width 0.6) (layer F.Cu) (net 16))
 (segment (start 140.335 130.175) (end 139.7 130.81) (width 0.6) (layer F.Cu) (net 16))
 (segment (start 140.335 127) (end 140.335 130.175) (width 0.6) (layer F.Cu) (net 16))
 (segment (start 139.065 125.73) (end 140.335 127) (width 0.6) (layer F.Cu) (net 16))
 (segment (start 139.065 118.745) (end 139.065 125.73) (width 0.6) (layer F.Cu) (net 16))
 (segment (start 137.7 117.38) (end 139.065 118.745) (width 0.6) (layer F.Cu) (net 16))
 (segment (start 136.525 117.38) (end 132.08 117.38) (width 0.6) (layer F.Cu) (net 16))
 (segment (start 109.855 129.54) (end 111.76 129.54) (width 1) (layer F.Cu) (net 17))
 (segment (start 116.84 109.22) (end 145.32 109.22) (width 1) (layer F.Cu) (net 17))
 (segment (start 114.3 111.76) (end 116.84 109.22) (width 1) (layer F.Cu) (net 17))
 (segment (start 114.3 127) (end 114.3 111.76) (width 1) (layer F.Cu) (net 17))
 (segment (start 111.76 129.54) (end 114.3 127) (width 1) (layer F.Cu) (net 17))
 (segment (start 145.32 114.3) (end 145.32 109.22) (width 1) (layer F.Cu) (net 17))
 (segment (start 131.285 128.27) (end 132.715 128.27) (width 0.6) (layer F.Cu) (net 56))
 (segment (start 132.715 133.35) (end 131.285 133.35) (width 0.6) (layer F.Cu) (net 56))
 (segment (start 133.35 132.715) (end 132.715 133.35) (width 0.6) (layer F.Cu) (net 56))
 (segment (start 133.35 128.905) (end 133.35 132.715) (width 0.6) (layer F.Cu) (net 56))
 (segment (start 132.715 128.27) (end 133.35 128.905) (width 0.6) (layer F.Cu) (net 56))
 (segment (start 131.285 133.35) (end 128.905 133.35) (width 0.6) (layer F.Cu) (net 56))
 (segment (start 131.285 129.54) (end 128.905 129.54) (width 0.6) (layer F.Cu) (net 56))
 (segment (start 128.905 128.27) (end 131.285 128.27) (width 0.6) (layer F.Cu) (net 56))
 (segment (start 128.905 129.54) (end 128.905 128.27) (width 0.6) (layer F.Cu) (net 56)))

